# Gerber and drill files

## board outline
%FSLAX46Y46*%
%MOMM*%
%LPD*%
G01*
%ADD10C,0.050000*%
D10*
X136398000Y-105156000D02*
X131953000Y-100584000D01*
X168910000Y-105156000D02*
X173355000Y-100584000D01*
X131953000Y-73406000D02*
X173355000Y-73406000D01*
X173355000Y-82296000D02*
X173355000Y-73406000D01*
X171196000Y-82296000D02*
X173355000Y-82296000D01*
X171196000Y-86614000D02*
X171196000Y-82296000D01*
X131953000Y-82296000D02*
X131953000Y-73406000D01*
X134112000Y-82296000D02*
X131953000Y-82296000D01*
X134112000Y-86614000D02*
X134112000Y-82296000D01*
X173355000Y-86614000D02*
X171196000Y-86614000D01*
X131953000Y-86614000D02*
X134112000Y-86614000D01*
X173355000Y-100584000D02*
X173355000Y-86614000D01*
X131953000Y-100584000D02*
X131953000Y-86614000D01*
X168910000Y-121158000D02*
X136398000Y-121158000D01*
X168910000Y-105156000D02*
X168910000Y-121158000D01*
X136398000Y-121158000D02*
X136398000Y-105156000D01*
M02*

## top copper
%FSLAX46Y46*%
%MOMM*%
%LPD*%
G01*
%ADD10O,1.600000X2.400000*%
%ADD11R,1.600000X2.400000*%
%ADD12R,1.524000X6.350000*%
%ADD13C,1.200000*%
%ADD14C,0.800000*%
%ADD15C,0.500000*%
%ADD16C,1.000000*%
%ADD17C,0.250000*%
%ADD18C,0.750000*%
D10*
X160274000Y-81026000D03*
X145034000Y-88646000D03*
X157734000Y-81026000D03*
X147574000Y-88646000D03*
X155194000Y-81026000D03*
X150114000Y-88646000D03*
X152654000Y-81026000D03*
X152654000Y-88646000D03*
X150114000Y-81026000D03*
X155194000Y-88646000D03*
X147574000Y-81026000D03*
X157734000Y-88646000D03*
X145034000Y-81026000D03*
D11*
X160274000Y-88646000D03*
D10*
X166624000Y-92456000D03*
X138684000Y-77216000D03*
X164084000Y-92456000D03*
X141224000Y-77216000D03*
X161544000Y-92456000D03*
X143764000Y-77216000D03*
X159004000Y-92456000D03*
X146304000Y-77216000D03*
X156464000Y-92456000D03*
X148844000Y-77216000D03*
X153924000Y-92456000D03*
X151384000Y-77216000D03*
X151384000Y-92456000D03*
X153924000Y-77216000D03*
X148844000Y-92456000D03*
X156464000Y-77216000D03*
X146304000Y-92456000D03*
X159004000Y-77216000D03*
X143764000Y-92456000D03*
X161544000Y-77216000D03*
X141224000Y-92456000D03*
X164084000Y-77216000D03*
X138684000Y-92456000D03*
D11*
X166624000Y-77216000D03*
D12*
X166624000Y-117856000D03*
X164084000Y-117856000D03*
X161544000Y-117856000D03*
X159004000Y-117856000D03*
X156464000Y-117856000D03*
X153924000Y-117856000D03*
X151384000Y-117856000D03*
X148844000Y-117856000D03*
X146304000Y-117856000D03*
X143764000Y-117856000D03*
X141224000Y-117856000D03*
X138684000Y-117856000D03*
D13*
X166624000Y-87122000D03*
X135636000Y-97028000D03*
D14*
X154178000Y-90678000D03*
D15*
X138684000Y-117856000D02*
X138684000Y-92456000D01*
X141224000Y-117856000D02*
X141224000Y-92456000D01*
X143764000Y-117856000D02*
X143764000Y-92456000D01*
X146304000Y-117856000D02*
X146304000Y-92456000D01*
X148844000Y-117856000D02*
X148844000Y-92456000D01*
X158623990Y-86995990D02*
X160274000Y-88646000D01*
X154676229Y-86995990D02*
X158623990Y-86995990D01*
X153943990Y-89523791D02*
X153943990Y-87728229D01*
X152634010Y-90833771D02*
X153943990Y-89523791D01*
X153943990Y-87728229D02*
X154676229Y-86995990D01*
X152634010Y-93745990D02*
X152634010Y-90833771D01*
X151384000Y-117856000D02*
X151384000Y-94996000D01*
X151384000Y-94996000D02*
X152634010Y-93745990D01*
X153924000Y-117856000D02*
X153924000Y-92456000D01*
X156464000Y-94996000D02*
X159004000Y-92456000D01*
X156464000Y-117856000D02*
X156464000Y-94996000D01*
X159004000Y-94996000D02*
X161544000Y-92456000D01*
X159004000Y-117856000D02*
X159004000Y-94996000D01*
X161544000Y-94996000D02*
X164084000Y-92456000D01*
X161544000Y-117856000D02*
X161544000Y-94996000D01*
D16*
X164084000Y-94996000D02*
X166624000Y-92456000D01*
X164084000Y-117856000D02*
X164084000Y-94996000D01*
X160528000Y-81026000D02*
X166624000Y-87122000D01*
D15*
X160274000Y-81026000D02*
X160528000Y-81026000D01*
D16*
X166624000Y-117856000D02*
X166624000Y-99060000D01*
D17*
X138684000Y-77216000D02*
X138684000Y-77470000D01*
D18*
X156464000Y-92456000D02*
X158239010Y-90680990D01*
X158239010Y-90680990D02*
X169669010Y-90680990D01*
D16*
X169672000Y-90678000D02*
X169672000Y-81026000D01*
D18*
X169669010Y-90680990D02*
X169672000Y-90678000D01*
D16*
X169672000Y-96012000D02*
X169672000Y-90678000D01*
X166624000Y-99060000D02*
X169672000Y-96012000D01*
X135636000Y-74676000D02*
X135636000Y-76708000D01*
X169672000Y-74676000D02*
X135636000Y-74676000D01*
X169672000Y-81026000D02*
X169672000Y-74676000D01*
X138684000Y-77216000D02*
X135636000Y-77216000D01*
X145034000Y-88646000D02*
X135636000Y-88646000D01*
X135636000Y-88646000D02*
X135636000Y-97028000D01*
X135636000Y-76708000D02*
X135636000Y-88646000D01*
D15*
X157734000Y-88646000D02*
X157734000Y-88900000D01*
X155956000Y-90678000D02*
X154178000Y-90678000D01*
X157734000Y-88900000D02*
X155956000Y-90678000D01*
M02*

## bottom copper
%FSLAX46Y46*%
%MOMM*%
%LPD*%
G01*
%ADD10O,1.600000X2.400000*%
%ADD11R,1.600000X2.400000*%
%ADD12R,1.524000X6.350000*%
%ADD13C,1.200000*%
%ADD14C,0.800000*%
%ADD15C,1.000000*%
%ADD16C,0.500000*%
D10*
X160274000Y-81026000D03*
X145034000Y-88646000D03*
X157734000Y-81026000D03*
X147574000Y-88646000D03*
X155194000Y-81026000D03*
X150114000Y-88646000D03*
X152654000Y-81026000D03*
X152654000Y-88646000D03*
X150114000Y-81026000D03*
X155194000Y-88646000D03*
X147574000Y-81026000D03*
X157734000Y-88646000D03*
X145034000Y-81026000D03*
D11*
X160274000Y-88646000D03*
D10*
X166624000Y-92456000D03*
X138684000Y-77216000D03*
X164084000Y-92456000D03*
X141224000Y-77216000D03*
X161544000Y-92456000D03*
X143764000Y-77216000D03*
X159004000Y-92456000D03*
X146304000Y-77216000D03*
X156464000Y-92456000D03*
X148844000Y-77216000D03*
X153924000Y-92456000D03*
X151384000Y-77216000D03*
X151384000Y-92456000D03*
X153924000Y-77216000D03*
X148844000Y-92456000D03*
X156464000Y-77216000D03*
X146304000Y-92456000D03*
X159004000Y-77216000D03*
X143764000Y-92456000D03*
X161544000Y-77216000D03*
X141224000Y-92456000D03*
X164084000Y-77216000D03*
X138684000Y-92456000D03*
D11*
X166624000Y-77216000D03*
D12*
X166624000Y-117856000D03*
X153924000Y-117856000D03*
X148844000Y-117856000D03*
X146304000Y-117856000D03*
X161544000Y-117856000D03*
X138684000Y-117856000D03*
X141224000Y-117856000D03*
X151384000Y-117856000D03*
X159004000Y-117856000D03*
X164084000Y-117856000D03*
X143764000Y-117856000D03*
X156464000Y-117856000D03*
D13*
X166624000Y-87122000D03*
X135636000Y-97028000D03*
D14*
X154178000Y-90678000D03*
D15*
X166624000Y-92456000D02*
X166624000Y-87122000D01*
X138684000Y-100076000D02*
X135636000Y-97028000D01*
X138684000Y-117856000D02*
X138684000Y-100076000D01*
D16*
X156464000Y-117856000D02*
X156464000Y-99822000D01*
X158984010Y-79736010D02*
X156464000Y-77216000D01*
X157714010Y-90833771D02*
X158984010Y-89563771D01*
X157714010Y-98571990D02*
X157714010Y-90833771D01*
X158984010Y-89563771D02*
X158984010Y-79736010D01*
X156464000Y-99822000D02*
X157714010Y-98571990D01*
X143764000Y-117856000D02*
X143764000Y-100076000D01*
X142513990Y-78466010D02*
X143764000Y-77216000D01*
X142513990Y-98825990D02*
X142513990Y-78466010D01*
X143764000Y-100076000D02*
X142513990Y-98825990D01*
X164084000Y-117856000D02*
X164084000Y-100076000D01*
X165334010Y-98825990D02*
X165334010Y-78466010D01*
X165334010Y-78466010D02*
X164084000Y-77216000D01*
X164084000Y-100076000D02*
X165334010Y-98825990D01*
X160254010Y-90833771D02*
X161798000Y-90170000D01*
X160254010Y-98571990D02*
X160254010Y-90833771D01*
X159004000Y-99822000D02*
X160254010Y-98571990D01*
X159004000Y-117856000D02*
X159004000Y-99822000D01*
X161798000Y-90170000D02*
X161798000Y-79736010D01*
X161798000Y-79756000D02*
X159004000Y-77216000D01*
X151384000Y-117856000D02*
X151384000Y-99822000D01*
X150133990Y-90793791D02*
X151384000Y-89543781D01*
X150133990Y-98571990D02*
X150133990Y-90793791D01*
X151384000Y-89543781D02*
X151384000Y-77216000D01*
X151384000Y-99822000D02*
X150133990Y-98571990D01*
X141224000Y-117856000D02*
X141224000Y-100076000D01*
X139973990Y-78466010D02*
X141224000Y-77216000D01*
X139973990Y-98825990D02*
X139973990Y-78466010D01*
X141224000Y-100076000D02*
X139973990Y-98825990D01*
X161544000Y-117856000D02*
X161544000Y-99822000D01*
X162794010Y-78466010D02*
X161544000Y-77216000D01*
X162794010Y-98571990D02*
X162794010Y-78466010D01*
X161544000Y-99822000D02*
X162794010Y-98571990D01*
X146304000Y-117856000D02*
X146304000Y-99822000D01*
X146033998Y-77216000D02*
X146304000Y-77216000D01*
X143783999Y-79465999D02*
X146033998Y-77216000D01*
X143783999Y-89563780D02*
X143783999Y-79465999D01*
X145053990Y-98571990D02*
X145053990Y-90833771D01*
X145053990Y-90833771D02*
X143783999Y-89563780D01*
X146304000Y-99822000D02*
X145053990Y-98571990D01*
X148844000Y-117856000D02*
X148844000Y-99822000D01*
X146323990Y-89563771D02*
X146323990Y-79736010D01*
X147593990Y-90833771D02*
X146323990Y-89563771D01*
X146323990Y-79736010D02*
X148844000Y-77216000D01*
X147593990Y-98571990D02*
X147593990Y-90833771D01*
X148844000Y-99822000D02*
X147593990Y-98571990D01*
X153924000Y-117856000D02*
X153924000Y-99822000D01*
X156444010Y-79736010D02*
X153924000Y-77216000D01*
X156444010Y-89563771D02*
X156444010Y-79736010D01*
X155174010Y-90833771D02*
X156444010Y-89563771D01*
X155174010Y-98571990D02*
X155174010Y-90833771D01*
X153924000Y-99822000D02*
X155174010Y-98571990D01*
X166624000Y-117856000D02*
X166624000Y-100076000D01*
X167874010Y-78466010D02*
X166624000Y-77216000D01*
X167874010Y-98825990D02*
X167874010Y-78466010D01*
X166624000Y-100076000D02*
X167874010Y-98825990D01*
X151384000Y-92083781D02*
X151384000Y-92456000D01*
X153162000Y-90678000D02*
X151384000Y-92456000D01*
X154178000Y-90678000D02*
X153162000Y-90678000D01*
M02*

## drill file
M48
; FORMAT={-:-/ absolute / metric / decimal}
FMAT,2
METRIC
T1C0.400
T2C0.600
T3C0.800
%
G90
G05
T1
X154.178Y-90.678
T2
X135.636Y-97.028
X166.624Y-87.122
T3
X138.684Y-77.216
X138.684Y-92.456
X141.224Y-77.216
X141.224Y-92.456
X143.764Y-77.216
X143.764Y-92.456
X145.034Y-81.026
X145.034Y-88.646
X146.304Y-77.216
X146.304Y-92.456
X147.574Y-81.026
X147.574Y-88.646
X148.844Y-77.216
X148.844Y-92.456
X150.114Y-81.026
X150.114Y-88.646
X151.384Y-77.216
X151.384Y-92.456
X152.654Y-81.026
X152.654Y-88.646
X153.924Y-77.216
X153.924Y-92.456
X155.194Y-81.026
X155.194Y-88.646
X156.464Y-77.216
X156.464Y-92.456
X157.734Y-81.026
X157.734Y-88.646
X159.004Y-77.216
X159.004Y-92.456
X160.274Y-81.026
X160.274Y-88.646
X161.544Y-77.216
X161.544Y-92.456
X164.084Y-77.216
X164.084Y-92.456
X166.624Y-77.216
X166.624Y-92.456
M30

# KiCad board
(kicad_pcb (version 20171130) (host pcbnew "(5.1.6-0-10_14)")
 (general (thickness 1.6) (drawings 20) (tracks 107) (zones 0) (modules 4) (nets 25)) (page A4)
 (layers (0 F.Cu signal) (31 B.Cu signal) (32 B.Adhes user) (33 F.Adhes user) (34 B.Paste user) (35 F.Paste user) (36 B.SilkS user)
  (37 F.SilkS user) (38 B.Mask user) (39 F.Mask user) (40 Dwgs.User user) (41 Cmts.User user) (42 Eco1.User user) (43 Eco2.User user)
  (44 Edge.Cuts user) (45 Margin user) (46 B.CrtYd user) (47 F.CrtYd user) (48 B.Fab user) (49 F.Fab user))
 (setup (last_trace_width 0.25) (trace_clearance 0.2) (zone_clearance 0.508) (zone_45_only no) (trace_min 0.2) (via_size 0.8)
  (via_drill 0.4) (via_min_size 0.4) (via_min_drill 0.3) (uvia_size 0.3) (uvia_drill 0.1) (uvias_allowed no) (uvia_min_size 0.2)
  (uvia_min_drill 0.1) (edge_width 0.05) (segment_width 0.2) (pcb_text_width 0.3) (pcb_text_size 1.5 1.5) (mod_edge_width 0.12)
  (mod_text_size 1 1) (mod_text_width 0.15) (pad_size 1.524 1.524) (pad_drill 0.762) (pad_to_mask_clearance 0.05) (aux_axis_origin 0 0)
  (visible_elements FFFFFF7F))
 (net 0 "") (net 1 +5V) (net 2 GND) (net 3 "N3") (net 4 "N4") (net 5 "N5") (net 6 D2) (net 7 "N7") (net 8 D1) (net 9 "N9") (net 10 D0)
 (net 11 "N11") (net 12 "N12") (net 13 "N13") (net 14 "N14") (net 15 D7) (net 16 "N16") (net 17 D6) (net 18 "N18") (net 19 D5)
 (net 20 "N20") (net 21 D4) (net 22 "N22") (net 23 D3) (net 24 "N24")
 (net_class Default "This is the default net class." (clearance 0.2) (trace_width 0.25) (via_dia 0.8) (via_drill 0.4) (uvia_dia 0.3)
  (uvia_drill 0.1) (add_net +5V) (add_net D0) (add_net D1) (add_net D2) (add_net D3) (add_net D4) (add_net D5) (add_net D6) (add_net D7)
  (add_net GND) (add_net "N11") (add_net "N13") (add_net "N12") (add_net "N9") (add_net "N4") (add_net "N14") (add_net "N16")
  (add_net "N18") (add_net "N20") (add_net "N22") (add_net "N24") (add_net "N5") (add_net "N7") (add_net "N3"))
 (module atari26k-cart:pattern (layer F.Cu) (at 152.654 105.41)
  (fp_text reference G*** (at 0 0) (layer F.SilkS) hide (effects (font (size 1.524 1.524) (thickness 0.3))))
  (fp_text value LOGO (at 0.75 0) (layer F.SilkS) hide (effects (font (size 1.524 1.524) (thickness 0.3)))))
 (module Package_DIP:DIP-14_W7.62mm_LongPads (layer B.Cu) (at 160.274 88.646 90)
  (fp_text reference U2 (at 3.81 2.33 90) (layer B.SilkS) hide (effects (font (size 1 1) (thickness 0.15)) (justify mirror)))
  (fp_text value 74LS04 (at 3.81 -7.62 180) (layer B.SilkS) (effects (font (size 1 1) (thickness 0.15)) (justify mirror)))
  (pad 14 thru_hole oval (at 7.62 0 90) (size 2.4 1.6) (drill 0.8) (layers *.Cu *.Mask) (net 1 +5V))
  (pad 7 thru_hole oval (at 0 -15.24 90) (size 2.4 1.6) (drill 0.8) (layers *.Cu *.Mask) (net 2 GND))
  (pad 13 thru_hole oval (at 7.62 -2.54 90) (size 2.4 1.6) (drill 0.8) (layers *.Cu *.Mask))
  (pad 6 thru_hole oval (at 0 -12.7 90) (size 2.4 1.6) (drill 0.8) (layers *.Cu *.Mask))
  (pad 12 thru_hole oval (at 7.62 -5.08 90) (size 2.4 1.6) (drill 0.8) (layers *.Cu *.Mask))
  (pad 5 thru_hole oval (at 0 -10.16 90) (size 2.4 1.6) (drill 0.8) (layers *.Cu *.Mask))
  (pad 11 thru_hole oval (at 7.62 -7.62 90) (size 2.4 1.6) (drill 0.8) (layers *.Cu *.Mask))
  (pad 4 thru_hole oval (at 0 -7.62 90) (size 2.4 1.6) (drill 0.8) (layers *.Cu *.Mask))
  (pad 10 thru_hole oval (at 7.62 -10.16 90) (size 2.4 1.6) (drill 0.8) (layers *.Cu *.Mask))
  (pad 3 thru_hole oval (at 0 -5.08 90) (size 2.4 1.6) (drill 0.8) (layers *.Cu *.Mask))
  (pad 9 thru_hole oval (at 7.62 -12.7 90) (size 2.4 1.6) (drill 0.8) (layers *.Cu *.Mask))
  (pad 2 thru_hole oval (at 0 -2.54 90) (size 2.4 1.6) (drill 0.8) (layers *.Cu *.Mask) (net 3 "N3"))
  (pad 8 thru_hole oval (at 7.62 -15.24 90) (size 2.4 1.6) (drill 0.8) (layers *.Cu *.Mask))
  (pad 1 thru_hole rect (at 0 0 90) (size 2.4 1.6) (drill 0.8) (layers *.Cu *.Mask) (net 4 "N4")))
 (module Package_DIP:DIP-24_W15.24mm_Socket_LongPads (layer F.Cu) (at 166.624 77.216 270)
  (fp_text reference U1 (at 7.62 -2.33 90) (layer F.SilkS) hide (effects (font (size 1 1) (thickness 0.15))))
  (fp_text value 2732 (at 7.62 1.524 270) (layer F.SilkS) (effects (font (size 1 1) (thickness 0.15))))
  (pad 24 thru_hole oval (at 15.24 0 270) (size 2.4 1.6) (drill 0.8) (layers *.Cu *.Mask) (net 1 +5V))
  (pad 12 thru_hole oval (at 0 27.94 270) (size 2.4 1.6) (drill 0.8) (layers *.Cu *.Mask) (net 2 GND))
  (pad 23 thru_hole oval (at 15.24 2.54 270) (size 2.4 1.6) (drill 0.8) (layers *.Cu *.Mask) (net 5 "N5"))
  (pad 11 thru_hole oval (at 0 25.4 270) (size 2.4 1.6) (drill 0.8) (layers *.Cu *.Mask) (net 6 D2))
  (pad 22 thru_hole oval (at 15.24 5.08 270) (size 2.4 1.6) (drill 0.8) (layers *.Cu *.Mask) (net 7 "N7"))
  (pad 10 thru_hole oval (at 0 22.86 270) (size 2.4 1.6) (drill 0.8) (layers *.Cu *.Mask) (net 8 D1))
  (pad 21 thru_hole oval (at 15.24 7.62 270) (size 2.4 1.6) (drill 0.8) (layers *.Cu *.Mask) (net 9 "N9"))
  (pad 9 thru_hole oval (at 0 20.32 270) (size 2.4 1.6) (drill 0.8) (layers *.Cu *.Mask) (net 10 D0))
  (pad 20 thru_hole oval (at 15.24 10.16 270) (size 2.4 1.6) (drill 0.8) (layers *.Cu *.Mask) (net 2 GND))
  (pad 8 thru_hole oval (at 0 17.78 270) (size 2.4 1.6) (drill 0.8) (layers *.Cu *.Mask) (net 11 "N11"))
  (pad 19 thru_hole oval (at 15.24 12.7 270) (size 2.4 1.6) (drill 0.8) (layers *.Cu *.Mask) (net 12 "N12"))
  (pad 7 thru_hole oval (at 0 15.24 270) (size 2.4 1.6) (drill 0.8) (layers *.Cu *.Mask) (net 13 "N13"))
  (pad 18 thru_hole oval (at 15.24 15.24 270) (size 2.4 1.6) (drill 0.8) (layers *.Cu *.Mask) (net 3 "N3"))
  (pad 6 thru_hole oval (at 0 12.7 270) (size 2.4 1.6) (drill 0.8) (layers *.Cu *.Mask) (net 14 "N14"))
  (pad 17 thru_hole oval (at 15.24 17.78 270) (size 2.4 1.6) (drill 0.8) (layers *.Cu *.Mask) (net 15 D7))
  (pad 5 thru_hole oval (at 0 10.16 270) (size 2.4 1.6) (drill 0.8) (layers *.Cu *.Mask) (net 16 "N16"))
  (pad 16 thru_hole oval (at 15.24 20.32 270) (size 2.4 1.6) (drill 0.8) (layers *.Cu *.Mask) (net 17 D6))
  (pad 4 thru_hole oval (at 0 7.62 270) (size 2.4 1.6) (drill 0.8) (layers *.Cu *.Mask) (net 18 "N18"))
  (pad 15 thru_hole oval (at 15.24 22.86 270) (size 2.4 1.6) (drill 0.8) (layers *.Cu *.Mask) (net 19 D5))
  (pad 3 thru_hole oval (at 0 5.08 270) (size 2.4 1.6) (drill 0.8) (layers *.Cu *.Mask) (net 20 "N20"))
  (pad 14 thru_hole oval (at 15.24 25.4 270) (size 2.4 1.6) (drill 0.8) (layers *.Cu *.Mask) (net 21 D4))
  (pad 2 thru_hole oval (at 0 2.54 270) (size 2.4 1.6) (drill 0.8) (layers *.Cu *.Mask) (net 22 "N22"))
  (pad 13 thru_hole oval (at 15.24 27.94 270) (size 2.4 1.6) (drill 0.8) (layers *.Cu *.Mask) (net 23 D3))
  (pad 1 thru_hole rect (at 0 0 270) (size 2.4 1.6) (drill 0.8) (layers *.Cu *.Mask) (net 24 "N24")))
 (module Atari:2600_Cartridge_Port (layer F.Cu) (at 138.176 114.808)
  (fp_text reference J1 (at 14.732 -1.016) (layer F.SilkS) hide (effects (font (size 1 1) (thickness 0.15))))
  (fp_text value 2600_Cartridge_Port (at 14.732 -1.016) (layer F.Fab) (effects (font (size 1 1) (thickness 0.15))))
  (pad A7 connect rect (at 28.448 3.048) (size 1.524 6.35) (layers B.Cu B.Mask) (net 24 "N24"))
  (pad A2 connect rect (at 15.748 3.048) (size 1.524 6.35) (layers B.Cu B.Mask) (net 14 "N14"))
  (pad A0 connect rect (at 10.668 3.048) (size 1.524 6.35) (layers B.Cu B.Mask) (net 11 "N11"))
  (pad D0 connect rect (at 8.128 3.048) (size 1.524 6.35) (layers B.Cu B.Mask) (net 10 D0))
  (pad A5 connect rect (at 23.368 3.048) (size 1.524 6.35) (layers B.Cu B.Mask) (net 20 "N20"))
  (pad GND connect rect (at 0.508 3.048) (size 1.524 6.35) (layers B.Cu B.Mask) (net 2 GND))
  (pad D2 connect rect (at 3.048 3.048) (size 1.524 6.35) (layers B.Cu B.Mask) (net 6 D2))
  (pad A1 connect rect (at 13.208 3.048) (size 1.524 6.35) (layers B.Cu B.Mask) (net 13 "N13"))
  (pad A4 connect rect (at 20.828 3.048) (size 1.524 6.35) (layers B.Cu B.Mask) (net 18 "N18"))
  (pad A6 connect rect (at 25.908 3.048) (size 1.524 6.35) (layers B.Cu B.Mask) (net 22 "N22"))
  (pad D1 connect rect (at 5.588 3.048) (size 1.524 6.35) (layers B.Cu B.Mask) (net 8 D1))
  (pad A3 connect rect (at 18.288 3.048) (size 1.524 6.35) (layers B.Cu B.Mask) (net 16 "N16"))
  (pad SGND connect rect (at 28.448 3.048) (size 1.524 6.35) (layers F.Cu F.Mask) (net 2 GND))
  (pad +5V connect rect (at 25.908 3.048) (size 1.524 6.35) (layers F.Cu F.Mask) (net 1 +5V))
  (pad A8 connect rect (at 23.368 3.048) (size 1.524 6.35) (layers F.Cu F.Mask) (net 5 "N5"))
  (pad A9 connect rect (at 20.828 3.048) (size 1.524 6.35) (layers F.Cu F.Mask) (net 7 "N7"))
  (pad A11 connect rect (at 18.288 3.048) (size 1.524 6.35) (layers F.Cu F.Mask) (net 9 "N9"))
  (pad A10 connect rect (at 15.748 3.048) (size 1.524 6.35) (layers F.Cu F.Mask) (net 12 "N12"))
  (pad A12 connect rect (at 13.208 3.048) (size 1.524 6.35) (layers F.Cu F.Mask) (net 4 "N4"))
  (pad D7 connect rect (at 10.668 3.048) (size 1.524 6.35) (layers F.Cu F.Mask) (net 15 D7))
  (pad D6 connect rect (at 8.128 3.048) (size 1.524 6.35) (layers F.Cu F.Mask) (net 17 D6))
  (pad D5 connect rect (at 5.588 3.048) (size 1.524 6.35) (layers F.Cu F.Mask) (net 19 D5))
  (pad D4 connect rect (at 3.048 3.048) (size 1.524 6.35) (layers F.Cu F.Mask) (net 21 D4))
  (pad D3 connect rect (at 0.508 3.048) (size 1.524 6.35) (layers F.Cu F.Mask) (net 23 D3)))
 (gr_line (start 136.398 105.156) (end 131.953 100.584) (layer Edge.Cuts) (width 0.05))
 (gr_line (start 168.91 105.156) (end 173.355 100.584) (layer Edge.Cuts) (width 0.05))
 (gr_line (start 131.953 73.406) (end 173.355 73.406) (layer Edge.Cuts) (width 0.05))
 (gr_line (start 173.355 82.296) (end 173.355 73.406) (layer Edge.Cuts) (width 0.05))
 (gr_line (start 171.196 82.296) (end 173.355 82.296) (layer Edge.Cuts) (width 0.05))
 (gr_line (start 171.196 86.614) (end 171.196 82.296) (layer Edge.Cuts) (width 0.05))
 (gr_line (start 131.953 82.296) (end 131.953 73.406) (layer Edge.Cuts) (width 0.05))
 (gr_line (start 134.112 82.296) (end 131.953 82.296) (layer Edge.Cuts) (width 0.05))
 (gr_line (start 134.112 86.614) (end 134.112 82.296) (layer Edge.Cuts) (width 0.05))
 (gr_line (start 173.355 86.614) (end 171.196 86.614) (layer Edge.Cuts) (width 0.05))
 (gr_line (start 131.953 86.614) (end 134.112 86.614) (layer Edge.Cuts) (width 0.05))
 (gr_line (start 173.355 100.584) (end 173.355 86.614) (layer Edge.Cuts) (width 0.05))
 (gr_line (start 131.953 100.584) (end 131.953 86.614) (layer Edge.Cuts) (width 0.05))
 (gr_line (start 168.91 121.158) (end 136.398 121.158) (layer Edge.Cuts) (width 0.05))
 (gr_line (start 168.91 105.156) (end 168.91 121.158) (layer Edge.Cuts) (width 0.05))
 (gr_line (start 136.398 121.158) (end 136.398 105.156) (layer Edge.Cuts) (width 0.05))
 (segment (start 138.684 117.856) (end 138.684 92.456) (width 0.5) (layer F.Cu) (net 23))
 (segment (start 141.224 117.856) (end 141.224 92.456) (width 0.5) (layer F.Cu) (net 21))
 (segment (start 143.764 117.856) (end 143.764 92.456) (width 0.5) (layer F.Cu) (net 19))
 (segment (start 146.304 117.856) (end 146.304 92.456) (width 0.5) (layer F.Cu) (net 17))
 (segment (start 148.844 117.856) (end 148.844 92.456) (width 0.5) (layer F.Cu) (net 15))
 (segment (start 158.62399 86.99599) (end 160.274 88.646) (width 0.5) (layer F.Cu) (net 4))
 (segment (start 154.676229 86.99599) (end 158.62399 86.99599) (width 0.5) (layer F.Cu) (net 4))
 (segment (start 153.94399 89.523791) (end 153.94399 87.728229) (width 0.5) (layer F.Cu) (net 4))
 (segment (start 152.63401 90.833771) (end 153.94399 89.523791) (width 0.5) (layer F.Cu) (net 4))
 (segment (start 153.94399 87.728229) (end 154.676229 86.99599) (width 0.5) (layer F.Cu) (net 4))
 (segment (start 152.63401 93.74599) (end 152.63401 90.833771) (width 0.5) (layer F.Cu) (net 4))
 (segment (start 151.384 117.856) (end 151.384 94.996) (width 0.5) (layer F.Cu) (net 4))
 (segment (start 151.384 94.996) (end 152.63401 93.74599) (width 0.5) (layer F.Cu) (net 4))
 (segment (start 153.924 117.856) (end 153.924 92.456) (width 0.5) (layer F.Cu) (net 12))
 (segment (start 156.464 94.996) (end 159.004 92.456) (width 0.5) (layer F.Cu) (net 9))
 (segment (start 156.464 117.856) (end 156.464 94.996) (width 0.5) (layer F.Cu) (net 9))
 (segment (start 159.004 94.996) (end 161.544 92.456) (width 0.5) (layer F.Cu) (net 7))
 (segment (start 159.004 117.856) (end 159.004 94.996) (width 0.5) (layer F.Cu) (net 7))
 (segment (start 161.544 94.996) (end 164.084 92.456) (width 0.5) (layer F.Cu) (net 5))
 (segment (start 161.544 117.856) (end 161.544 94.996) (width 0.5) (layer F.Cu) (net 5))
 (segment (start 164.084 94.996) (end 166.624 92.456) (width 1) (layer F.Cu) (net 1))
 (segment (start 164.084 117.856) (end 164.084 94.996) (width 1) (layer F.Cu) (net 1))
 (via (at 166.624 87.122) (size 1.2) (drill 0.6) (layers F.Cu B.Cu) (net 1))
 (segment (start 166.624 92.456) (end 166.624 87.122) (width 1) (layer B.Cu) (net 1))
 (segment (start 160.528 81.026) (end 166.624 87.122) (width 1) (layer F.Cu) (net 1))
 (segment (start 160.274 81.026) (end 160.528 81.026) (width 0.5) (layer F.Cu) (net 1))
 (segment (start 166.624 117.856) (end 166.624 99.06) (width 1) (layer F.Cu) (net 2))
 (segment (start 138.684 77.216) (end 138.684 77.47) (width 0.25) (layer F.Cu) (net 2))
 (segment (start 156.464 92.456) (end 158.23901 90.68099) (width 0.75) (layer F.Cu) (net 2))
 (segment (start 158.23901 90.68099) (end 169.66901 90.68099) (width 0.75) (layer F.Cu) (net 2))
 (segment (start 169.672 90.678) (end 169.672 81.026) (width 1) (layer F.Cu) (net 2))
 (segment (start 169.66901 90.68099) (end 169.672 90.678) (width 0.75) (layer F.Cu) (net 2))
 (via (at 135.636 97.028) (size 1.2) (drill 0.6) (layers F.Cu B.Cu) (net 2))
 (segment (start 169.672 96.012) (end 169.672 90.678) (width 1) (layer F.Cu) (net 2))
 (segment (start 166.624 99.06) (end 169.672 96.012) (width 1) (layer F.Cu) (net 2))
 (segment (start 135.636 74.676) (end 135.636 76.708) (width 1) (layer F.Cu) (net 2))
 (segment (start 138.684 100.076) (end 135.636 97.028) (width 1) (layer B.Cu) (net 2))
 (segment (start 138.684 117.856) (end 138.684 100.076) (width 1) (layer B.Cu) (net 2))
 (segment (start 169.672 74.676) (end 135.636 74.676) (width 1) (layer F.Cu) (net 2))
 (segment (start 169.672 81.026) (end 169.672 74.676) (width 1) (layer F.Cu) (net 2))
 (segment (start 138.684 77.216) (end 135.636 77.216) (width 1) (layer F.Cu) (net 2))
 (segment (start 145.034 88.646) (end 135.636 88.646) (width 1) (layer F.Cu) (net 2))
 (segment (start 135.636 88.646) (end 135.636 97.028) (width 1) (layer F.Cu) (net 2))
 (segment (start 135.636 76.708) (end 135.636 88.646) (width 1) (layer F.Cu) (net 2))
 (segment (start 156.464 117.856) (end 156.464 99.822) (width 0.5) (layer B.Cu) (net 16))
 (segment (start 158.98401 79.73601) (end 156.464 77.216) (width 0.5) (layer B.Cu) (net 16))
 (segment (start 157.71401 90.833771) (end 158.98401 89.563771) (width 0.5) (layer B.Cu) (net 16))
 (segment (start 157.71401 98.57199) (end 157.71401 90.833771) (width 0.5) (layer B.Cu) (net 16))
 (segment (start 158.98401 89.563771) (end 158.98401 79.73601) (width 0.5) (layer B.Cu) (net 16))
 (segment (start 156.464 99.822) (end 157.71401 98.57199) (width 0.5) (layer B.Cu) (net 16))
 (segment (start 143.764 117.856) (end 143.764 100.076) (width 0.5) (layer B.Cu) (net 8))
 (segment (start 142.51399 78.46601) (end 143.764 77.216) (width 0.5) (layer B.Cu) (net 8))
 (segment (start 142.51399 98.82599) (end 142.51399 78.46601) (width 0.5) (layer B.Cu) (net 8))
 (segment (start 143.764 100.076) (end 142.51399 98.82599) (width 0.5) (layer B.Cu) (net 8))
 (segment (start 164.084 117.856) (end 164.084 100.076) (width 0.5) (layer B.Cu) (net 22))
 (segment (start 165.33401 98.82599) (end 165.33401 78.46601) (width 0.5) (layer B.Cu) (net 22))
 (segment (start 165.33401 78.46601) (end 164.084 77.216) (width 0.5) (layer B.Cu) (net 22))
 (segment (start 164.084 100.076) (end 165.33401 98.82599) (width 0.5) (layer B.Cu) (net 22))
 (segment (start 160.25401 90.833771) (end 161.798 90.17) (width 0.5) (layer B.Cu) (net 18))
 (segment (start 160.25401 98.57199) (end 160.25401 90.833771) (width 0.5) (layer B.Cu) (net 18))
 (segment (start 159.004 99.822) (end 160.25401 98.57199) (width 0.5) (layer B.Cu) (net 18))
 (segment (start 159.004 117.856) (end 159.004 99.822) (width 0.5) (layer B.Cu) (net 18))
 (segment (start 161.798 90.17) (end 161.798 79.73601) (width 0.5) (layer B.Cu) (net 18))
 (segment (start 161.798 79.756) (end 159.004 77.216) (width 0.5) (layer B.Cu) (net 18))
 (segment (start 151.384 117.856) (end 151.384 99.822) (width 0.5) (layer B.Cu) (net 13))
 (segment (start 150.13399 90.793791) (end 151.384 89.543781) (width 0.5) (layer B.Cu) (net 13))
 (segment (start 150.13399 98.57199) (end 150.13399 90.793791) (width 0.5) (layer B.Cu) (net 13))
 (segment (start 151.384 89.543781) (end 151.384 77.216) (width 0.5) (layer B.Cu) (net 13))
 (segment (start 151.384 99.822) (end 150.13399 98.57199) (width 0.5) (layer B.Cu) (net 13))
 (segment (start 141.224 117.856) (end 141.224 100.076) (width 0.5) (layer B.Cu) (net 6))
 (segment (start 139.97399 78.46601) (end 141.224 77.216) (width 0.5) (layer B.Cu) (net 6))
 (segment (start 139.97399 98.82599) (end 139.97399 78.46601) (width 0.5) (layer B.Cu) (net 6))
 (segment (start 141.224 100.076) (end 139.97399 98.82599) (width 0.5) (layer B.Cu) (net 6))
 (segment (start 161.544 117.856) (end 161.544 99.822) (width 0.5) (layer B.Cu) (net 20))
 (segment (start 162.79401 78.46601) (end 161.544 77.216) (width 0.5) (layer B.Cu) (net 20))
 (segment (start 162.79401 98.57199) (end 162.79401 78.46601) (width 0.5) (layer B.Cu) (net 20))
 (segment (start 161.544 99.822) (end 162.79401 98.57199) (width 0.5) (layer B.Cu) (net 20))
 (segment (start 146.304 117.856) (end 146.304 99.822) (width 0.5) (layer B.Cu) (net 10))
 (segment (start 146.033998 77.216) (end 146.304 77.216) (width 0.5) (layer B.Cu) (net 10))
 (segment (start 143.783999 79.465999) (end 146.033998 77.216) (width 0.5) (layer B.Cu) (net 10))
 (segment (start 143.783999 89.56378) (end 143.783999 79.465999) (width 0.5) (layer B.Cu) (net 10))
 (segment (start 145.05399 98.57199) (end 145.05399 90.833771) (width 0.5) (layer B.Cu) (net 10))
 (segment (start 145.05399 90.833771) (end 143.783999 89.56378) (width 0.5) (layer B.Cu) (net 10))
 (segment (start 146.304 99.822) (end 145.05399 98.57199) (width 0.5) (layer B.Cu) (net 10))
 (segment (start 148.844 117.856) (end 148.844 99.822) (width 0.5) (layer B.Cu) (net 11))
 (segment (start 146.32399 89.563771) (end 146.32399 79.73601) (width 0.5) (layer B.Cu) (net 11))
 (segment (start 147.59399 90.833771) (end 146.32399 89.563771) (width 0.5) (layer B.Cu) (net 11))
 (segment (start 146.32399 79.73601) (end 148.844 77.216) (width 0.5) (layer B.Cu) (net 11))
 (segment (start 147.59399 98.57199) (end 147.59399 90.833771) (width 0.5) (layer B.Cu) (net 11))
 (segment (start 148.844 99.822) (end 147.59399 98.57199) (width 0.5) (layer B.Cu) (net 11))
 (segment (start 153.924 117.856) (end 153.924 99.822) (width 0.5) (layer B.Cu) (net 14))
 (segment (start 156.44401 79.73601) (end 153.924 77.216) (width 0.5) (layer B.Cu) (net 14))
 (segment (start 156.44401 89.563771) (end 156.44401 79.73601) (width 0.5) (layer B.Cu) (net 14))
 (segment (start 155.17401 90.833771) (end 156.44401 89.563771) (width 0.5) (layer B.Cu) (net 14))
 (segment (start 155.17401 98.57199) (end 155.17401 90.833771) (width 0.5) (layer B.Cu) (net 14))
 (segment (start 153.924 99.822) (end 155.17401 98.57199) (width 0.5) (layer B.Cu) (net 14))
 (segment (start 166.624 117.856) (end 166.624 100.076) (width 0.5) (layer B.Cu) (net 24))
 (segment (start 167.87401 78.46601) (end 166.624 77.216) (width 0.5) (layer B.Cu) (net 24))
 (segment (start 167.87401 98.82599) (end 167.87401 78.46601) (width 0.5) (layer B.Cu) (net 24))
 (segment (start 166.624 100.076) (end 167.87401 98.82599) (width 0.5) (layer B.Cu) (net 24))
 (segment (start 151.384 92.083781) (end 151.384 92.456) (width 0.5) (layer B.Cu) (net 3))
 (segment (start 157.734 88.646) (end 157.734 88.9) (width 0.5) (layer F.Cu) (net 3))
 (via (at 154.178 90.678) (size 0.8) (drill 0.4) (layers F.Cu B.Cu) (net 3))
 (segment (start 155.956 90.678) (end 154.178 90.678) (width 0.5) (layer F.Cu) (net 3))
 (segment (start 157.734 88.9) (end 155.956 90.678) (width 0.5) (layer F.Cu) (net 3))
 (segment (start 153.162 90.678) (end 151.384 92.456) (width 0.5) (layer B.Cu) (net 3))
 (segment (start 154.178 90.678) (end 153.162 90.678) (width 0.5) (layer B.Cu) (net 3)))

